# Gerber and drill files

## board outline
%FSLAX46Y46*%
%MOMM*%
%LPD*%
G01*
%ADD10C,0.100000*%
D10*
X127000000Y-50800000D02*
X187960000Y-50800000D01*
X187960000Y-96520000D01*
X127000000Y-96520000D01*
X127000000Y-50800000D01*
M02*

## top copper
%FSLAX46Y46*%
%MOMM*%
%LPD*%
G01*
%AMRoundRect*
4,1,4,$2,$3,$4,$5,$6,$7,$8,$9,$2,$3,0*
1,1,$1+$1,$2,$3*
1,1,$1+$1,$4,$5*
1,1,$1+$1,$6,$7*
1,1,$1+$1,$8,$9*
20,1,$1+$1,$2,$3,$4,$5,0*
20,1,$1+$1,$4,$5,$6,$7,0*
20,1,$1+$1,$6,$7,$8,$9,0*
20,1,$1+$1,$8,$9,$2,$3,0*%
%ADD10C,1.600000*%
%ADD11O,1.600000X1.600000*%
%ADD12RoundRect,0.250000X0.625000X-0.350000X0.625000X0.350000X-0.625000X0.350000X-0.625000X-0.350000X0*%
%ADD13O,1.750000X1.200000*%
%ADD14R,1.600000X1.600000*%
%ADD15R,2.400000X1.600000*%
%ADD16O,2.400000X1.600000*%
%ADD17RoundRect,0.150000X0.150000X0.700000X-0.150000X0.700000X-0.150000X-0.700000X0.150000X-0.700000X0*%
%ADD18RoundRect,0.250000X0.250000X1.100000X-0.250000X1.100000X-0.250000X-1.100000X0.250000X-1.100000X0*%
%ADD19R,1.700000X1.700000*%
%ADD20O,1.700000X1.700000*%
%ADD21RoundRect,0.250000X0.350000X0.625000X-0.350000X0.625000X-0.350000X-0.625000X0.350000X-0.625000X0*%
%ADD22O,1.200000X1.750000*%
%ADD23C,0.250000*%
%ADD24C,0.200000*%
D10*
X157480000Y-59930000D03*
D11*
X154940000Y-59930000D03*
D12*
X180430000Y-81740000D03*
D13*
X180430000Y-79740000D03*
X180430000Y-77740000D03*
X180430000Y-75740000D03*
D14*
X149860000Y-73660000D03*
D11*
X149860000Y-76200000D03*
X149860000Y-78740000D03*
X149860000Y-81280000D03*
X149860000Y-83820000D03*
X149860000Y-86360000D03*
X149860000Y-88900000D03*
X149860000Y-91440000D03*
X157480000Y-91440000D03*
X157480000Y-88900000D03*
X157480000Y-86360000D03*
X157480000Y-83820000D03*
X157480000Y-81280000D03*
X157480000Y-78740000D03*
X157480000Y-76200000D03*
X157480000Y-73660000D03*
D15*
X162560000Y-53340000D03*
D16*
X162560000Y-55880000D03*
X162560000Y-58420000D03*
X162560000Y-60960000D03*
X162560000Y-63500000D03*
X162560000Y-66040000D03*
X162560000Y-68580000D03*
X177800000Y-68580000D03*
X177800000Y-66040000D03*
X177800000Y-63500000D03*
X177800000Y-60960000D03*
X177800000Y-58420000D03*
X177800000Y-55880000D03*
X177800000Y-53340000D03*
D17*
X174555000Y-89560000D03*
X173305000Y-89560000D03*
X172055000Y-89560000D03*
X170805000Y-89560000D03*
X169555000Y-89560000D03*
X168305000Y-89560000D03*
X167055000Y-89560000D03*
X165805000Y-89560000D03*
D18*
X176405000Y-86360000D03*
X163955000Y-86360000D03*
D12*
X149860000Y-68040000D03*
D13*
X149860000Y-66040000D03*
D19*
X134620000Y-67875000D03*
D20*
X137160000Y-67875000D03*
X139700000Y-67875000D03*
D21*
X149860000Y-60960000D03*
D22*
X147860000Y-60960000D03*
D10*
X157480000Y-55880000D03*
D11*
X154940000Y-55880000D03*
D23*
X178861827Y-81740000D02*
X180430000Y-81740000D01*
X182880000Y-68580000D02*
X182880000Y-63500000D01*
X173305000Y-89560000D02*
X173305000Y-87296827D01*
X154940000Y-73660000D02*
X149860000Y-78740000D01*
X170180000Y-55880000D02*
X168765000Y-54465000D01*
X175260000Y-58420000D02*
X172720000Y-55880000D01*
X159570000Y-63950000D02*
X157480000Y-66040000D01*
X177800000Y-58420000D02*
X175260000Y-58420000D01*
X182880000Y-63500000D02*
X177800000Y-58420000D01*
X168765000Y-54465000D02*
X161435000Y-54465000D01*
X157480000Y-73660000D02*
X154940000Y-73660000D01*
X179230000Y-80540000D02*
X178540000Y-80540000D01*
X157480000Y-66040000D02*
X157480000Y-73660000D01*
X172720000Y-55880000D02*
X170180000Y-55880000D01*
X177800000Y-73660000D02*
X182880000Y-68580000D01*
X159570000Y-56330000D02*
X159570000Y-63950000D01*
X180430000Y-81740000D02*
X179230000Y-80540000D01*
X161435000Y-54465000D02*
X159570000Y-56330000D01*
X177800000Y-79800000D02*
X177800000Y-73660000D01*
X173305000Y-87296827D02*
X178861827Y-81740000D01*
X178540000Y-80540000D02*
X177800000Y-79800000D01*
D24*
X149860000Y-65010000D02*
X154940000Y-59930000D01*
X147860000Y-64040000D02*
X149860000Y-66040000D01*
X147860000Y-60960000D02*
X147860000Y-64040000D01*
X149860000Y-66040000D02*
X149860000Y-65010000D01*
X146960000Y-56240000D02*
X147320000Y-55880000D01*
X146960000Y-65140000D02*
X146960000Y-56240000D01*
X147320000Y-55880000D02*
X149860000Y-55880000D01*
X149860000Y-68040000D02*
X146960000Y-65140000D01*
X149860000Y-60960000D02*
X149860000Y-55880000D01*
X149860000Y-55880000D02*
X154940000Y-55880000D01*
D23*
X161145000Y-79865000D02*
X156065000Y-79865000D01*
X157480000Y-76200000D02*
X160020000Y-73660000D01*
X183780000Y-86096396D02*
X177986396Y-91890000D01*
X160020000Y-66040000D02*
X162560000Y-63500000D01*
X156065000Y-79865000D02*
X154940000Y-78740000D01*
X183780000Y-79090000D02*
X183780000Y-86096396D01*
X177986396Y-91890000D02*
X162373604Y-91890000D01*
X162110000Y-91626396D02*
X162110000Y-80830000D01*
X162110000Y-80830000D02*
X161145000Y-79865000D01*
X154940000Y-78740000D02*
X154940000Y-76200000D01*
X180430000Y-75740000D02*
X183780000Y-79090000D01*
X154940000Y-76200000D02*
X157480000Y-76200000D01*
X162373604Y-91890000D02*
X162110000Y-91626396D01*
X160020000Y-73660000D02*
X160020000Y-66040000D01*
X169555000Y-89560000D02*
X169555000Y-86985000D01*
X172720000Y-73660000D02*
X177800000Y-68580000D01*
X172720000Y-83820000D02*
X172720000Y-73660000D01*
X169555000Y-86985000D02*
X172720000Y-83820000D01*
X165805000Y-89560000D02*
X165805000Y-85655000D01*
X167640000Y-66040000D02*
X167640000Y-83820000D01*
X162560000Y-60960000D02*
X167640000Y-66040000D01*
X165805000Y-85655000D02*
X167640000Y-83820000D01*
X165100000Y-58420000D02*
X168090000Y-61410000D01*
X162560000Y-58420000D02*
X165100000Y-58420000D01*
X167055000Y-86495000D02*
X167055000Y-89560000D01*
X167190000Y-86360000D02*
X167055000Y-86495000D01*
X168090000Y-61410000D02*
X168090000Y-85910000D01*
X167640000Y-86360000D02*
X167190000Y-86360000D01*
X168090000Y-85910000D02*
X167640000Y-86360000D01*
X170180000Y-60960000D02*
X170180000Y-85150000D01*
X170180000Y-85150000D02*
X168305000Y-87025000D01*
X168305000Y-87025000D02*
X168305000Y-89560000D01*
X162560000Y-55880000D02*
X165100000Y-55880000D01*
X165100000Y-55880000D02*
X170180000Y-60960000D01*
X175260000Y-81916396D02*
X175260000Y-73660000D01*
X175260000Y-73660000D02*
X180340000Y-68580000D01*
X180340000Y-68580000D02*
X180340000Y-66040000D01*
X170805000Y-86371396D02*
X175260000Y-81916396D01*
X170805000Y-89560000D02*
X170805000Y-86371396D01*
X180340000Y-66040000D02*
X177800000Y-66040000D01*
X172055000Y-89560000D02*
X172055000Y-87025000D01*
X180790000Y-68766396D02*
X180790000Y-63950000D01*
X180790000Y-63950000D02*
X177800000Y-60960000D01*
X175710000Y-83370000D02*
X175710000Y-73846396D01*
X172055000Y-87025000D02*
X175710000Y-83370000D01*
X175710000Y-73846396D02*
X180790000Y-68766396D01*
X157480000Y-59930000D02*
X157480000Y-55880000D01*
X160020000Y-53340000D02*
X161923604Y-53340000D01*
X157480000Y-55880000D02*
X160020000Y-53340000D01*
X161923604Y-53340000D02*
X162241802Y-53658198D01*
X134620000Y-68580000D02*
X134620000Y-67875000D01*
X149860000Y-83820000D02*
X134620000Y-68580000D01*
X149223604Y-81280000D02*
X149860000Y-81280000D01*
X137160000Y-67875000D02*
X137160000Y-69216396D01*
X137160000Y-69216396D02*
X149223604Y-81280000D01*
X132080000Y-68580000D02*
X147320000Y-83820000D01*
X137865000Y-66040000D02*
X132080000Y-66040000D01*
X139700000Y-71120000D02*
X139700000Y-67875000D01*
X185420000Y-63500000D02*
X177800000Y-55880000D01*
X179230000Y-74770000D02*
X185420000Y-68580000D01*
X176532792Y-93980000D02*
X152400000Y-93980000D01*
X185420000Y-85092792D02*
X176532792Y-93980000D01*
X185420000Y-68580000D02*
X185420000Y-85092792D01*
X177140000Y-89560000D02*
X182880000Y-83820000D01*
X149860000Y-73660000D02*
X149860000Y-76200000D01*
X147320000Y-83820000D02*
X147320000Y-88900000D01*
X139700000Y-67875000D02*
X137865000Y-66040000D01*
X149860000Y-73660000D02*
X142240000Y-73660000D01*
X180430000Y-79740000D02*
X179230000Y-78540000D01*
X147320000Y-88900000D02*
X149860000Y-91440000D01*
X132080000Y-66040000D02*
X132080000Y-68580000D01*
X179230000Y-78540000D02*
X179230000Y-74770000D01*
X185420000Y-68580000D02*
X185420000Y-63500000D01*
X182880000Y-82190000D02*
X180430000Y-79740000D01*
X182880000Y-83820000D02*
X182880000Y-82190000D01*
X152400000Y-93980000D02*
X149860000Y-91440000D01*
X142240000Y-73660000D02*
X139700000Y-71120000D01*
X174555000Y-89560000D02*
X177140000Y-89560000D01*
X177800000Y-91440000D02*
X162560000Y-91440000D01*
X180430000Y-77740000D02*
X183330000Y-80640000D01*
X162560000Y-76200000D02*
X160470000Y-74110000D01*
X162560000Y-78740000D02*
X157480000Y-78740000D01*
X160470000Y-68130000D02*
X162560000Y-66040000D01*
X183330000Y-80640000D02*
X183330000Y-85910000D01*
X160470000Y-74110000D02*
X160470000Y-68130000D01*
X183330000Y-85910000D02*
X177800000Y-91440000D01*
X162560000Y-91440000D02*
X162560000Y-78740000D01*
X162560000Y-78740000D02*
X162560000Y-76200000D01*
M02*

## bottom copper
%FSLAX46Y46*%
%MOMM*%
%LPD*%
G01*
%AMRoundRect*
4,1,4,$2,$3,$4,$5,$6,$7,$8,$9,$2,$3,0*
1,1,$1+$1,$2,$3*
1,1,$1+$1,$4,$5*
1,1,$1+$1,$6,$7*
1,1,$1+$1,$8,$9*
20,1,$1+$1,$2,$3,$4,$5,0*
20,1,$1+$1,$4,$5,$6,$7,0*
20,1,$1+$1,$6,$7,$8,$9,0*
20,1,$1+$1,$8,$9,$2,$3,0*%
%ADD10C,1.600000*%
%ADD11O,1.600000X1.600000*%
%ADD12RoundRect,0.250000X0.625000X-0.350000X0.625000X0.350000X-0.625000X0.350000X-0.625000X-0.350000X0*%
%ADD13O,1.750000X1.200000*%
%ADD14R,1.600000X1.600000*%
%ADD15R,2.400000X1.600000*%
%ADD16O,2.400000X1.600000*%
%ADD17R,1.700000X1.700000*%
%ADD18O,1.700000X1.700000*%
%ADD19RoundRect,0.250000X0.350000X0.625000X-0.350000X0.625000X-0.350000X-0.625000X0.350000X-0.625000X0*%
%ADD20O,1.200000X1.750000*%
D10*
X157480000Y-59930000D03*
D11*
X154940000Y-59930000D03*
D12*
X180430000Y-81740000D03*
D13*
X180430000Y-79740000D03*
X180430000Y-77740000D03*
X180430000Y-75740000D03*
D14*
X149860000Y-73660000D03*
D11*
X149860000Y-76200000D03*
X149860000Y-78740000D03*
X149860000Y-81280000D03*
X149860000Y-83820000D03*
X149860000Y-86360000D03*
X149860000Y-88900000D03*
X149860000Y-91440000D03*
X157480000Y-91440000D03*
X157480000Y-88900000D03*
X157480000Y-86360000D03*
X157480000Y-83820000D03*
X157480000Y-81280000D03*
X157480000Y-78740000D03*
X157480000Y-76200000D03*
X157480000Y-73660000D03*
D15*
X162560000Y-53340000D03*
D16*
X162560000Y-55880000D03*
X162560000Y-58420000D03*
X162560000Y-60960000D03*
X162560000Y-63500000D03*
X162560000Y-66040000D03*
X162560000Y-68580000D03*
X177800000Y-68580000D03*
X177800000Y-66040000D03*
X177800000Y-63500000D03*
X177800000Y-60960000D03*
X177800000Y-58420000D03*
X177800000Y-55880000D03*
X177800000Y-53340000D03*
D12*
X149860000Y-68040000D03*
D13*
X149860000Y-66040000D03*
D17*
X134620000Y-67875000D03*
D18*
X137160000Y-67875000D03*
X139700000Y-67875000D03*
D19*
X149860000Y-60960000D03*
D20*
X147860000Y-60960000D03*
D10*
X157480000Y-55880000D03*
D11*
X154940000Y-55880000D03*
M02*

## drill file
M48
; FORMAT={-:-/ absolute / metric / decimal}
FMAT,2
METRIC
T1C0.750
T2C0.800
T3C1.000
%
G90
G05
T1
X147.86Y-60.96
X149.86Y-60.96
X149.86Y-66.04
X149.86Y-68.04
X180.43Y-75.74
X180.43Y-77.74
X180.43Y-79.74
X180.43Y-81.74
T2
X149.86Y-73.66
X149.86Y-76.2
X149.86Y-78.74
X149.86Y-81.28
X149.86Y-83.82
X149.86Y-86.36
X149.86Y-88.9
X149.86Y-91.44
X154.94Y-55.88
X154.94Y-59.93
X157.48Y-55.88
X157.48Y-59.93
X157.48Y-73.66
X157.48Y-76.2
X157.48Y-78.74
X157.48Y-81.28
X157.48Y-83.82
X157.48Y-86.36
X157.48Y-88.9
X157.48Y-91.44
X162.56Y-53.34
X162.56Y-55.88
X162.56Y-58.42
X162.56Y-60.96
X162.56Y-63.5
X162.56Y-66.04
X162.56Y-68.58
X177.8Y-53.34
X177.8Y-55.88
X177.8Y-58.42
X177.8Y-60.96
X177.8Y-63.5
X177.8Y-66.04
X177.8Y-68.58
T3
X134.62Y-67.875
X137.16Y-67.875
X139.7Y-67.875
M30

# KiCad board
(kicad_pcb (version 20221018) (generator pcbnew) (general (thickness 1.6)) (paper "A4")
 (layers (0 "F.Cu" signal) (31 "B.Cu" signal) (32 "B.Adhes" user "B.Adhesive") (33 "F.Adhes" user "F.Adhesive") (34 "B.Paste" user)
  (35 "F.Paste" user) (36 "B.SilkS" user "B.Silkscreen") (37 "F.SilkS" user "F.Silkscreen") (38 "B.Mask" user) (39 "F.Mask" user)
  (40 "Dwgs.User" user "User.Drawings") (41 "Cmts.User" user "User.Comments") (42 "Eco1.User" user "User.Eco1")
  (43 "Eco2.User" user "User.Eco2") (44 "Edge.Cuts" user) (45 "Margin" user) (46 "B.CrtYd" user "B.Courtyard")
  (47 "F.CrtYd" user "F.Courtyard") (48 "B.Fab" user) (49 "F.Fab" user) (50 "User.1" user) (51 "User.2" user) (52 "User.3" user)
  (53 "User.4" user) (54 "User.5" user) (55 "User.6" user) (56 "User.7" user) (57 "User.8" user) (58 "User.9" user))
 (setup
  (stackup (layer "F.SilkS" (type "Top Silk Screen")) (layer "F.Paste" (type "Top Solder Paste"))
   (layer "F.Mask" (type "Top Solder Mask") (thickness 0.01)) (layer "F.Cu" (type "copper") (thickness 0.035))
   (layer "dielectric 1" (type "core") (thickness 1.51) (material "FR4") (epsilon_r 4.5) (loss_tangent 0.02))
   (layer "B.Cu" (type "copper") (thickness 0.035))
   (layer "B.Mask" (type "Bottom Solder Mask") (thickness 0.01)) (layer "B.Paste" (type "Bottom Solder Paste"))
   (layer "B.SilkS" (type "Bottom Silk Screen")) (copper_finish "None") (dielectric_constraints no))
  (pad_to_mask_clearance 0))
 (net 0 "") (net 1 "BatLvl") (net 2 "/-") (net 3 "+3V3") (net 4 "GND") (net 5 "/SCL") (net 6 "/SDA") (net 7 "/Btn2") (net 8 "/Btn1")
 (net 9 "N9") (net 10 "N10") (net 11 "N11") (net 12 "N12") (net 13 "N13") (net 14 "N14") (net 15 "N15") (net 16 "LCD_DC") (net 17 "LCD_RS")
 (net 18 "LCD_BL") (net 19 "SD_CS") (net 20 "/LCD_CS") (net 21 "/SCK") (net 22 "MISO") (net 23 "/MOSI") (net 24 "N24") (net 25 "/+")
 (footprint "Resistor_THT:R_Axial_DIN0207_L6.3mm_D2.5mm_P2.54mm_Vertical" (layer "F.Cu") (at 157.48 59.93 180)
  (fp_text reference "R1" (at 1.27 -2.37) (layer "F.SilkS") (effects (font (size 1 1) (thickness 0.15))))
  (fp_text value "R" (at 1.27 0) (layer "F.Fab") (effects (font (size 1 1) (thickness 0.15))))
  (pad "1" thru_hole circle (at 0 0 180) (size 1.6 1.6) (drill 0.8) (layers "*.Cu" "*.Mask") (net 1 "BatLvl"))
  (pad "2" thru_hole oval (at 2.54 0 180) (size 1.6 1.6) (drill 0.8) (layers "*.Cu" "*.Mask") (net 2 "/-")))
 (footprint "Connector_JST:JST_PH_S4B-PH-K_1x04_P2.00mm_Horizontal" (layer "F.Cu") (at 180.43 81.74 90)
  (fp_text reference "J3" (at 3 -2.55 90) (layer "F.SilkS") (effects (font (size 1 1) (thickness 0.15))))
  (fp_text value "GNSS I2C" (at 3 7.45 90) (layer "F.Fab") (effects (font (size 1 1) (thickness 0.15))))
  (pad "1" thru_hole roundrect (at 0 0 90) (size 1.2 1.75) (drill 0.75) (layers "*.Cu" "*.Mask") (roundrect_rratio 0.208333) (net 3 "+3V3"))
  (pad "2" thru_hole oval (at 2 0 90) (size 1.2 1.75) (drill 0.75) (layers "*.Cu" "*.Mask") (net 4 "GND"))
  (pad "3" thru_hole oval (at 4 0 90) (size 1.2 1.75) (drill 0.75) (layers "*.Cu" "*.Mask") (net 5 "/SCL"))
  (pad "4" thru_hole oval (at 6 0 90) (size 1.2 1.75) (drill 0.75) (layers "*.Cu" "*.Mask") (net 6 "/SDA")))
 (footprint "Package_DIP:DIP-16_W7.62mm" (layer "F.Cu") (at 149.86 73.66)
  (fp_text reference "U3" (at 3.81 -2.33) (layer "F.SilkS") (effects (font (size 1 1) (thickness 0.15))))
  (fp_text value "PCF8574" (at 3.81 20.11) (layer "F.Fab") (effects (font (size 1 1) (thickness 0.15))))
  (pad "1" thru_hole rect (at 0 0) (size 1.6 1.6) (drill 0.8) (layers "*.Cu" "*.Mask") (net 4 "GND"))
  (pad "2" thru_hole oval (at 0 2.54) (size 1.6 1.6) (drill 0.8) (layers "*.Cu" "*.Mask") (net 4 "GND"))
  (pad "3" thru_hole oval (at 0 5.08) (size 1.6 1.6) (drill 0.8) (layers "*.Cu" "*.Mask") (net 3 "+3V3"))
  (pad "4" thru_hole oval (at 0 7.62) (size 1.6 1.6) (drill 0.8) (layers "*.Cu" "*.Mask") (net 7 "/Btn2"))
  (pad "5" thru_hole oval (at 0 10.16) (size 1.6 1.6) (drill 0.8) (layers "*.Cu" "*.Mask") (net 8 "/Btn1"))
  (pad "6" thru_hole oval (at 0 12.7) (size 1.6 1.6) (drill 0.8) (layers "*.Cu" "*.Mask") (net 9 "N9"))
  (pad "7" thru_hole oval (at 0 15.24) (size 1.6 1.6) (drill 0.8) (layers "*.Cu" "*.Mask") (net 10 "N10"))
  (pad "8" thru_hole oval (at 0 17.78) (size 1.6 1.6) (drill 0.8) (layers "*.Cu" "*.Mask") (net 4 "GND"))
  (pad "9" thru_hole oval (at 7.62 17.78) (size 1.6 1.6) (drill 0.8) (layers "*.Cu" "*.Mask") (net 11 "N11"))
  (pad "10" thru_hole oval (at 7.62 15.24) (size 1.6 1.6) (drill 0.8) (layers "*.Cu" "*.Mask") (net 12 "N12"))
  (pad "11" thru_hole oval (at 7.62 12.7) (size 1.6 1.6) (drill 0.8) (layers "*.Cu" "*.Mask") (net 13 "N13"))
  (pad "12" thru_hole oval (at 7.62 10.16) (size 1.6 1.6) (drill 0.8) (layers "*.Cu" "*.Mask") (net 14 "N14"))
  (pad "13" thru_hole oval (at 7.62 7.62) (size 1.6 1.6) (drill 0.8) (layers "*.Cu" "*.Mask") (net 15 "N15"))
  (pad "14" thru_hole oval (at 7.62 5.08) (size 1.6 1.6) (drill 0.8) (layers "*.Cu" "*.Mask") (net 5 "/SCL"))
  (pad "15" thru_hole oval (at 7.62 2.54) (size 1.6 1.6) (drill 0.8) (layers "*.Cu" "*.Mask") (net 6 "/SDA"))
  (pad "16" thru_hole oval (at 7.62 0) (size 1.6 1.6) (drill 0.8) (layers "*.Cu" "*.Mask") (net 3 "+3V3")))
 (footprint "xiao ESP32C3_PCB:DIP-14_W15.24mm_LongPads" (layer "F.Cu") (at 162.56 53.34)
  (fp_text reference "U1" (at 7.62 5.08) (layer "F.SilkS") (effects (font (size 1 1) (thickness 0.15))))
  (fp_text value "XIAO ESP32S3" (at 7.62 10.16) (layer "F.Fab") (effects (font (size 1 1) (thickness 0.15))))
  (pad "1" thru_hole rect (at 0 0) (size 2.4 1.6) (drill 0.8) (layers "*.Cu" "*.Mask") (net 1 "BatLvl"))
  (pad "2" thru_hole oval (at 0 2.54) (size 2.4 1.6) (drill 0.8) (layers "*.Cu" "*.Mask") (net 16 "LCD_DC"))
  (pad "3" thru_hole oval (at 0 5.08) (size 2.4 1.6) (drill 0.8) (layers "*.Cu" "*.Mask") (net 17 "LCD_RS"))
  (pad "4" thru_hole oval (at 0 7.62) (size 2.4 1.6) (drill 0.8) (layers "*.Cu" "*.Mask") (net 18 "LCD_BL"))
  (pad "5" thru_hole oval (at 0 10.16) (size 2.4 1.6) (drill 0.8) (layers "*.Cu" "*.Mask") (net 6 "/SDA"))
  (pad "6" thru_hole oval (at 0 12.7) (size 2.4 1.6) (drill 0.8) (layers "*.Cu" "*.Mask") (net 5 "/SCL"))
  (pad "7" thru_hole oval (at 0 15.24) (size 2.4 1.6) (drill 0.8) (layers "*.Cu" "*.Mask") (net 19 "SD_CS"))
  (pad "8" thru_hole oval (at 15.24 15.24) (size 2.4 1.6) (drill 0.8) (layers "*.Cu" "*.Mask") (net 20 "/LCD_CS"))
  (pad "9" thru_hole oval (at 15.24 12.7) (size 2.4 1.6) (drill 0.8) (layers "*.Cu" "*.Mask") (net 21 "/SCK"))
  (pad "10" thru_hole oval (at 15.24 10.16) (size 2.4 1.6) (drill 0.8) (layers "*.Cu" "*.Mask") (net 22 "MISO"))
  (pad "11" thru_hole oval (at 15.24 7.62) (size 2.4 1.6) (drill 0.8) (layers "*.Cu" "*.Mask") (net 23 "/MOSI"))
  (pad "12" thru_hole oval (at 15.24 5.08) (size 2.4 1.6) (drill 0.8) (layers "*.Cu" "*.Mask") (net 3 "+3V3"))
  (pad "13" thru_hole oval (at 15.24 2.54) (size 2.4 1.6) (drill 0.8) (layers "*.Cu" "*.Mask") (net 4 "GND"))
  (pad "14" thru_hole oval (at 15.24 0) (size 2.4 1.6) (drill 0.8) (layers "*.Cu" "*.Mask") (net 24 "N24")))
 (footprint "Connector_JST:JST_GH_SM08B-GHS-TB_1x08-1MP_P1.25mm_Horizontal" (layer "F.Cu") (at 170.18 87.71 180)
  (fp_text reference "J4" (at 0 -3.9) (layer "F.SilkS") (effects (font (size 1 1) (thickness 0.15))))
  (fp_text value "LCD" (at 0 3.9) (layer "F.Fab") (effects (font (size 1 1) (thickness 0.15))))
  (pad "1" smd roundrect (at -4.375 -1.85 180) (size 0.6 1.7) (layers "F.Cu" "F.Paste" "F.Mask") (roundrect_rratio 0.25) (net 4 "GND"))
  (pad "2" smd roundrect (at -3.125 -1.85 180) (size 0.6 1.7) (layers "F.Cu" "F.Paste" "F.Mask") (roundrect_rratio 0.25) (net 3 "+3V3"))
  (pad "3" smd roundrect (at -1.875 -1.85 180) (size 0.6 1.7) (layers "F.Cu" "F.Paste" "F.Mask") (roundrect_rratio 0.25) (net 23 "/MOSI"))
  (pad "4" smd roundrect (at -0.625 -1.85 180) (size 0.6 1.7) (layers "F.Cu" "F.Paste" "F.Mask") (roundrect_rratio 0.25) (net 21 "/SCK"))
  (pad "5" smd roundrect (at 0.625 -1.85 180) (size 0.6 1.7) (layers "F.Cu" "F.Paste" "F.Mask") (roundrect_rratio 0.25) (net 20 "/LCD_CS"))
  (pad "6" smd roundrect (at 1.875 -1.85 180) (size 0.6 1.7) (layers "F.Cu" "F.Paste" "F.Mask") (roundrect_rratio 0.25) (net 16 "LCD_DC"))
  (pad "7" smd roundrect (at 3.125 -1.85 180) (size 0.6 1.7) (layers "F.Cu" "F.Paste" "F.Mask") (roundrect_rratio 0.25) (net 17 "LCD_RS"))
  (pad "8" smd roundrect (at 4.375 -1.85 180) (size 0.6 1.7) (layers "F.Cu" "F.Paste" "F.Mask") (roundrect_rratio 0.25) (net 18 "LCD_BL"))
  (pad "MP" smd roundrect (at -6.225 1.35 180) (size 1 2.7) (layers "F.Cu" "F.Paste" "F.Mask") (roundrect_rratio 0.25))
  (pad "MP" smd roundrect (at 6.225 1.35 180) (size 1 2.7) (layers "F.Cu" "F.Paste" "F.Mask") (roundrect_rratio 0.25)))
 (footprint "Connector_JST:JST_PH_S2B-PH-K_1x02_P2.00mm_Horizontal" (layer "F.Cu") (at 149.86 68.04 90)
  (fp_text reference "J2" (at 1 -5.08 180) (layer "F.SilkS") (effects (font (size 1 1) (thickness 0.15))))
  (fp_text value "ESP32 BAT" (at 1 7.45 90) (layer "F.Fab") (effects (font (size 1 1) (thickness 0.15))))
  (pad "1" thru_hole roundrect (at 0 0 90) (size 1.2 1.75) (drill 0.75) (layers "*.Cu" "*.Mask") (roundrect_rratio 0.208333) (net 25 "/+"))
  (pad "2" thru_hole oval (at 2 0 90) (size 1.2 1.75) (drill 0.75) (layers "*.Cu" "*.Mask") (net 2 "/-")))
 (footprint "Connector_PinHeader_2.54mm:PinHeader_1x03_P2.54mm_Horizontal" (layer "F.Cu") (at 134.62 67.875 90)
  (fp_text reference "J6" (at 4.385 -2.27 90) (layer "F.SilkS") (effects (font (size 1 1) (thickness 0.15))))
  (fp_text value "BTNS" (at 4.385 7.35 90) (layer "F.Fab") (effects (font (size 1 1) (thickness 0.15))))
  (pad "1" thru_hole rect (at 0 0 90) (size 1.7 1.7) (drill 1) (layers "*.Cu" "*.Mask") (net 8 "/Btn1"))
  (pad "2" thru_hole oval (at 0 2.54 90) (size 1.7 1.7) (drill 1) (layers "*.Cu" "*.Mask") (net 7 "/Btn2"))
  (pad "3" thru_hole oval (at 0 5.08 90) (size 1.7 1.7) (drill 1) (layers "*.Cu" "*.Mask") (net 4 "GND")))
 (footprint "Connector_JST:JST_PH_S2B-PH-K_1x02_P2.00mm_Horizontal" (layer "F.Cu") (at 149.86 60.96 180)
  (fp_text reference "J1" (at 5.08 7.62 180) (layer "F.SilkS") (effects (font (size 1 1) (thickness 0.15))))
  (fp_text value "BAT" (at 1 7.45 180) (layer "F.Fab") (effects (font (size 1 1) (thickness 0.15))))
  (pad "1" thru_hole roundrect (at 0 0 180) (size 1.2 1.75) (drill 0.75) (layers "*.Cu" "*.Mask") (roundrect_rratio 0.208333) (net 25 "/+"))
  (pad "2" thru_hole oval (at 2 0 180) (size 1.2 1.75) (drill 0.75) (layers "*.Cu" "*.Mask") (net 2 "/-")))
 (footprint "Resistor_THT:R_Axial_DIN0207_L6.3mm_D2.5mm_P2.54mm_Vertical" (layer "F.Cu") (at 157.48 55.88 180)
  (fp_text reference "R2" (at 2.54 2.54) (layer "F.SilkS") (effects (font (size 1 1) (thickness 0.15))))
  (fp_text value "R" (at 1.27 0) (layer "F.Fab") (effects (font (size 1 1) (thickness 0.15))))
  (pad "1" thru_hole circle (at 0 0 180) (size 1.6 1.6) (drill 0.8) (layers "*.Cu" "*.Mask") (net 1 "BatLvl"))
  (pad "2" thru_hole oval (at 2.54 0 180) (size 1.6 1.6) (drill 0.8) (layers "*.Cu" "*.Mask") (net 25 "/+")))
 (gr_rect (start 127 50.8) (end 187.96 96.52) (stroke (width 0.1) (type default)) (fill none) (layer "Edge.Cuts"))
 (segment (start 178.861827 81.74) (end 180.43 81.74) (width 0.25) (layer "F.Cu") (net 3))
 (segment (start 182.88 68.58) (end 182.88 63.5) (width 0.25) (layer "F.Cu") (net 3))
 (segment (start 173.305 89.56) (end 173.305 87.296827) (width 0.25) (layer "F.Cu") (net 3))
 (segment (start 154.94 73.66) (end 149.86 78.74) (width 0.25) (layer "F.Cu") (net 3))
 (segment (start 170.18 55.88) (end 168.765 54.465) (width 0.25) (layer "F.Cu") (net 3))
 (segment (start 175.26 58.42) (end 172.72 55.88) (width 0.25) (layer "F.Cu") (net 3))
 (segment (start 159.57 63.95) (end 157.48 66.04) (width 0.25) (layer "F.Cu") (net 3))
 (segment (start 177.8 58.42) (end 175.26 58.42) (width 0.25) (layer "F.Cu") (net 3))
 (segment (start 182.88 63.5) (end 177.8 58.42) (width 0.25) (layer "F.Cu") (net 3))
 (segment (start 168.765 54.465) (end 161.435 54.465) (width 0.25) (layer "F.Cu") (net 3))
 (segment (start 157.48 73.66) (end 154.94 73.66) (width 0.25) (layer "F.Cu") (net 3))
 (segment (start 179.23 80.54) (end 178.54 80.54) (width 0.25) (layer "F.Cu") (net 3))
 (segment (start 157.48 66.04) (end 157.48 73.66) (width 0.25) (layer "F.Cu") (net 3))
 (segment (start 172.72 55.88) (end 170.18 55.88) (width 0.25) (layer "F.Cu") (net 3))
 (segment (start 177.8 73.66) (end 182.88 68.58) (width 0.25) (layer "F.Cu") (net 3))
 (segment (start 159.57 56.33) (end 159.57 63.95) (width 0.25) (layer "F.Cu") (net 3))
 (segment (start 180.43 81.74) (end 179.23 80.54) (width 0.25) (layer "F.Cu") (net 3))
 (segment (start 161.435 54.465) (end 159.57 56.33) (width 0.25) (layer "F.Cu") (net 3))
 (segment (start 177.8 79.8) (end 177.8 73.66) (width 0.25) (layer "F.Cu") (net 3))
 (segment (start 173.305 87.296827) (end 178.861827 81.74) (width 0.25) (layer "F.Cu") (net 3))
 (segment (start 178.54 80.54) (end 177.8 79.8) (width 0.25) (layer "F.Cu") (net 3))
 (segment (start 149.86 65.01) (end 154.94 59.93) (width 0.2) (layer "F.Cu") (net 2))
 (segment (start 147.86 64.04) (end 149.86 66.04) (width 0.2) (layer "F.Cu") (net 2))
 (segment (start 147.86 60.96) (end 147.86 64.04) (width 0.2) (layer "F.Cu") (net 2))
 (segment (start 149.86 66.04) (end 149.86 65.01) (width 0.2) (layer "F.Cu") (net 2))
 (segment (start 146.96 56.24) (end 147.32 55.88) (width 0.2) (layer "F.Cu") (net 25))
 (segment (start 146.96 65.14) (end 146.96 56.24) (width 0.2) (layer "F.Cu") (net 25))
 (segment (start 147.32 55.88) (end 149.86 55.88) (width 0.2) (layer "F.Cu") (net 25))
 (segment (start 149.86 68.04) (end 146.96 65.14) (width 0.2) (layer "F.Cu") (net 25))
 (segment (start 149.86 60.96) (end 149.86 55.88) (width 0.2) (layer "F.Cu") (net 25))
 (segment (start 149.86 55.88) (end 154.94 55.88) (width 0.2) (layer "F.Cu") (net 25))
 (segment (start 161.145 79.865) (end 156.065 79.865) (width 0.25) (layer "F.Cu") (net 6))
 (segment (start 157.48 76.2) (end 160.02 73.66) (width 0.25) (layer "F.Cu") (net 6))
 (segment (start 183.78 86.096396) (end 177.986396 91.89) (width 0.25) (layer "F.Cu") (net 6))
 (segment (start 160.02 66.04) (end 162.56 63.5) (width 0.25) (layer "F.Cu") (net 6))
 (segment (start 156.065 79.865) (end 154.94 78.74) (width 0.25) (layer "F.Cu") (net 6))
 (segment (start 183.78 79.09) (end 183.78 86.096396) (width 0.25) (layer "F.Cu") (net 6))
 (segment (start 177.986396 91.89) (end 162.373604 91.89) (width 0.25) (layer "F.Cu") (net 6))
 (segment (start 162.11 91.626396) (end 162.11 80.83) (width 0.25) (layer "F.Cu") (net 6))
 (segment (start 162.11 80.83) (end 161.145 79.865) (width 0.25) (layer "F.Cu") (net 6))
 (segment (start 154.94 78.74) (end 154.94 76.2) (width 0.25) (layer "F.Cu") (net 6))
 (segment (start 180.43 75.74) (end 183.78 79.09) (width 0.25) (layer "F.Cu") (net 6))
 (segment (start 154.94 76.2) (end 157.48 76.2) (width 0.25) (layer "F.Cu") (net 6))
 (segment (start 162.373604 91.89) (end 162.11 91.626396) (width 0.25) (layer "F.Cu") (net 6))
 (segment (start 160.02 73.66) (end 160.02 66.04) (width 0.25) (layer "F.Cu") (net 6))
 (segment (start 169.555 89.56) (end 169.555 86.985) (width 0.25) (layer "F.Cu") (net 20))
 (segment (start 172.72 73.66) (end 177.8 68.58) (width 0.25) (layer "F.Cu") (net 20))
 (segment (start 172.72 83.82) (end 172.72 73.66) (width 0.25) (layer "F.Cu") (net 20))
 (segment (start 169.555 86.985) (end 172.72 83.82) (width 0.25) (layer "F.Cu") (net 20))
 (segment (start 165.805 89.56) (end 165.805 85.655) (width 0.25) (layer "F.Cu") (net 18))
 (segment (start 167.64 66.04) (end 167.64 83.82) (width 0.25) (layer "F.Cu") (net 18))
 (segment (start 162.56 60.96) (end 167.64 66.04) (width 0.25) (layer "F.Cu") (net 18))
 (segment (start 165.805 85.655) (end 167.64 83.82) (width 0.25) (layer "F.Cu") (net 18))
 (segment (start 165.1 58.42) (end 168.09 61.41) (width 0.25) (layer "F.Cu") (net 17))
 (segment (start 162.56 58.42) (end 165.1 58.42) (width 0.25) (layer "F.Cu") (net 17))
 (segment (start 167.055 86.495) (end 167.055 89.56) (width 0.25) (layer "F.Cu") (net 17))
 (segment (start 167.19 86.36) (end 167.055 86.495) (width 0.25) (layer "F.Cu") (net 17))
 (segment (start 168.09 61.41) (end 168.09 85.91) (width 0.25) (layer "F.Cu") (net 17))
 (segment (start 167.64 86.36) (end 167.19 86.36) (width 0.25) (layer "F.Cu") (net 17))
 (segment (start 168.09 85.91) (end 167.64 86.36) (width 0.25) (layer "F.Cu") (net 17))
 (segment (start 170.18 60.96) (end 170.18 85.15) (width 0.25) (layer "F.Cu") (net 16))
 (segment (start 170.18 85.15) (end 168.305 87.025) (width 0.25) (layer "F.Cu") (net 16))
 (segment (start 168.305 87.025) (end 168.305 89.56) (width 0.25) (layer "F.Cu") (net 16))
 (segment (start 162.56 55.88) (end 165.1 55.88) (width 0.25) (layer "F.Cu") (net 16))
 (segment (start 165.1 55.88) (end 170.18 60.96) (width 0.25) (layer "F.Cu") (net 16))
 (segment (start 175.26 81.916396) (end 175.26 73.66) (width 0.25) (layer "F.Cu") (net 21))
 (segment (start 175.26 73.66) (end 180.34 68.58) (width 0.25) (layer "F.Cu") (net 21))
 (segment (start 180.34 68.58) (end 180.34 66.04) (width 0.25) (layer "F.Cu") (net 21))
 (segment (start 170.805 86.371396) (end 175.26 81.916396) (width 0.25) (layer "F.Cu") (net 21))
 (segment (start 170.805 89.56) (end 170.805 86.371396) (width 0.25) (layer "F.Cu") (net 21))
 (segment (start 180.34 66.04) (end 177.8 66.04) (width 0.25) (layer "F.Cu") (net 21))
 (segment (start 172.055 89.56) (end 172.055 87.025) (width 0.25) (layer "F.Cu") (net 23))
 (segment (start 180.79 68.766396) (end 180.79 63.95) (width 0.25) (layer "F.Cu") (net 23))
 (segment (start 180.79 63.95) (end 177.8 60.96) (width 0.25) (layer "F.Cu") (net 23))
 (segment (start 175.71 83.37) (end 175.71 73.846396) (width 0.25) (layer "F.Cu") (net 23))
 (segment (start 172.055 87.025) (end 175.71 83.37) (width 0.25) (layer "F.Cu") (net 23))
 (segment (start 175.71 73.846396) (end 180.79 68.766396) (width 0.25) (layer "F.Cu") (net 23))
 (segment (start 157.48 59.93) (end 157.48 55.88) (width 0.25) (layer "F.Cu") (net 1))
 (segment (start 160.02 53.34) (end 161.923604 53.34) (width 0.25) (layer "F.Cu") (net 1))
 (segment (start 157.48 55.88) (end 160.02 53.34) (width 0.25) (layer "F.Cu") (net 1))
 (segment (start 161.923604 53.34) (end 162.241802 53.658198) (width 0.25) (layer "F.Cu") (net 1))
 (segment (start 134.62 68.58) (end 134.62 67.875) (width 0.25) (layer "F.Cu") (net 8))
 (segment (start 149.86 83.82) (end 134.62 68.58) (width 0.25) (layer "F.Cu") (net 8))
 (segment (start 149.223604 81.28) (end 149.86 81.28) (width 0.25) (layer "F.Cu") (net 7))
 (segment (start 137.16 67.875) (end 137.16 69.216396) (width 0.25) (layer "F.Cu") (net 7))
 (segment (start 137.16 69.216396) (end 149.223604 81.28) (width 0.25) (layer "F.Cu") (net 7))
 (segment (start 132.08 68.58) (end 147.32 83.82) (width 0.25) (layer "F.Cu") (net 4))
 (segment (start 137.865 66.04) (end 132.08 66.04) (width 0.25) (layer "F.Cu") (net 4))
 (segment (start 139.7 71.12) (end 139.7 67.875) (width 0.25) (layer "F.Cu") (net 4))
 (segment (start 185.42 63.5) (end 177.8 55.88) (width 0.25) (layer "F.Cu") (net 4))
 (segment (start 179.23 74.77) (end 185.42 68.58) (width 0.25) (layer "F.Cu") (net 4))
 (segment (start 176.532792 93.98) (end 152.4 93.98) (width 0.25) (layer "F.Cu") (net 4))
 (segment (start 185.42 85.092792) (end 176.532792 93.98) (width 0.25) (layer "F.Cu") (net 4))
 (segment (start 185.42 68.58) (end 185.42 85.092792) (width 0.25) (layer "F.Cu") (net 4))
 (segment (start 177.14 89.56) (end 182.88 83.82) (width 0.25) (layer "F.Cu") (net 4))
 (segment (start 149.86 73.66) (end 149.86 76.2) (width 0.25) (layer "F.Cu") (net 4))
 (segment (start 147.32 83.82) (end 147.32 88.9) (width 0.25) (layer "F.Cu") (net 4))
 (segment (start 139.7 67.875) (end 137.865 66.04) (width 0.25) (layer "F.Cu") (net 4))
 (segment (start 149.86 73.66) (end 142.24 73.66) (width 0.25) (layer "F.Cu") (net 4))
 (segment (start 180.43 79.74) (end 179.23 78.54) (width 0.25) (layer "F.Cu") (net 4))
 (segment (start 147.32 88.9) (end 149.86 91.44) (width 0.25) (layer "F.Cu") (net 4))
 (segment (start 132.08 66.04) (end 132.08 68.58) (width 0.25) (layer "F.Cu") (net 4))
 (segment (start 179.23 78.54) (end 179.23 74.77) (width 0.25) (layer "F.Cu") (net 4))
 (segment (start 185.42 68.58) (end 185.42 63.5) (width 0.25) (layer "F.Cu") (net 4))
 (segment (start 182.88 82.19) (end 180.43 79.74) (width 0.25) (layer "F.Cu") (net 4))
 (segment (start 182.88 83.82) (end 182.88 82.19) (width 0.25) (layer "F.Cu") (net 4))
 (segment (start 152.4 93.98) (end 149.86 91.44) (width 0.25) (layer "F.Cu") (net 4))
 (segment (start 142.24 73.66) (end 139.7 71.12) (width 0.25) (layer "F.Cu") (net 4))
 (segment (start 174.555 89.56) (end 177.14 89.56) (width 0.25) (layer "F.Cu") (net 4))
 (segment (start 177.8 91.44) (end 162.56 91.44) (width 0.25) (layer "F.Cu") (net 5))
 (segment (start 180.43 77.74) (end 183.33 80.64) (width 0.25) (layer "F.Cu") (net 5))
 (segment (start 162.56 76.2) (end 160.47 74.11) (width 0.25) (layer "F.Cu") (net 5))
 (segment (start 162.56 78.74) (end 157.48 78.74) (width 0.25) (layer "F.Cu") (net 5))
 (segment (start 160.47 68.13) (end 162.56 66.04) (width 0.25) (layer "F.Cu") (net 5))
 (segment (start 183.33 80.64) (end 183.33 85.91) (width 0.25) (layer "F.Cu") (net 5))
 (segment (start 160.47 74.11) (end 160.47 68.13) (width 0.25) (layer "F.Cu") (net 5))
 (segment (start 183.33 85.91) (end 177.8 91.44) (width 0.25) (layer "F.Cu") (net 5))
 (segment (start 162.56 91.44) (end 162.56 78.74) (width 0.25) (layer "F.Cu") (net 5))
 (segment (start 162.56 78.74) (end 162.56 76.2) (width 0.25) (layer "F.Cu") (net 5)))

